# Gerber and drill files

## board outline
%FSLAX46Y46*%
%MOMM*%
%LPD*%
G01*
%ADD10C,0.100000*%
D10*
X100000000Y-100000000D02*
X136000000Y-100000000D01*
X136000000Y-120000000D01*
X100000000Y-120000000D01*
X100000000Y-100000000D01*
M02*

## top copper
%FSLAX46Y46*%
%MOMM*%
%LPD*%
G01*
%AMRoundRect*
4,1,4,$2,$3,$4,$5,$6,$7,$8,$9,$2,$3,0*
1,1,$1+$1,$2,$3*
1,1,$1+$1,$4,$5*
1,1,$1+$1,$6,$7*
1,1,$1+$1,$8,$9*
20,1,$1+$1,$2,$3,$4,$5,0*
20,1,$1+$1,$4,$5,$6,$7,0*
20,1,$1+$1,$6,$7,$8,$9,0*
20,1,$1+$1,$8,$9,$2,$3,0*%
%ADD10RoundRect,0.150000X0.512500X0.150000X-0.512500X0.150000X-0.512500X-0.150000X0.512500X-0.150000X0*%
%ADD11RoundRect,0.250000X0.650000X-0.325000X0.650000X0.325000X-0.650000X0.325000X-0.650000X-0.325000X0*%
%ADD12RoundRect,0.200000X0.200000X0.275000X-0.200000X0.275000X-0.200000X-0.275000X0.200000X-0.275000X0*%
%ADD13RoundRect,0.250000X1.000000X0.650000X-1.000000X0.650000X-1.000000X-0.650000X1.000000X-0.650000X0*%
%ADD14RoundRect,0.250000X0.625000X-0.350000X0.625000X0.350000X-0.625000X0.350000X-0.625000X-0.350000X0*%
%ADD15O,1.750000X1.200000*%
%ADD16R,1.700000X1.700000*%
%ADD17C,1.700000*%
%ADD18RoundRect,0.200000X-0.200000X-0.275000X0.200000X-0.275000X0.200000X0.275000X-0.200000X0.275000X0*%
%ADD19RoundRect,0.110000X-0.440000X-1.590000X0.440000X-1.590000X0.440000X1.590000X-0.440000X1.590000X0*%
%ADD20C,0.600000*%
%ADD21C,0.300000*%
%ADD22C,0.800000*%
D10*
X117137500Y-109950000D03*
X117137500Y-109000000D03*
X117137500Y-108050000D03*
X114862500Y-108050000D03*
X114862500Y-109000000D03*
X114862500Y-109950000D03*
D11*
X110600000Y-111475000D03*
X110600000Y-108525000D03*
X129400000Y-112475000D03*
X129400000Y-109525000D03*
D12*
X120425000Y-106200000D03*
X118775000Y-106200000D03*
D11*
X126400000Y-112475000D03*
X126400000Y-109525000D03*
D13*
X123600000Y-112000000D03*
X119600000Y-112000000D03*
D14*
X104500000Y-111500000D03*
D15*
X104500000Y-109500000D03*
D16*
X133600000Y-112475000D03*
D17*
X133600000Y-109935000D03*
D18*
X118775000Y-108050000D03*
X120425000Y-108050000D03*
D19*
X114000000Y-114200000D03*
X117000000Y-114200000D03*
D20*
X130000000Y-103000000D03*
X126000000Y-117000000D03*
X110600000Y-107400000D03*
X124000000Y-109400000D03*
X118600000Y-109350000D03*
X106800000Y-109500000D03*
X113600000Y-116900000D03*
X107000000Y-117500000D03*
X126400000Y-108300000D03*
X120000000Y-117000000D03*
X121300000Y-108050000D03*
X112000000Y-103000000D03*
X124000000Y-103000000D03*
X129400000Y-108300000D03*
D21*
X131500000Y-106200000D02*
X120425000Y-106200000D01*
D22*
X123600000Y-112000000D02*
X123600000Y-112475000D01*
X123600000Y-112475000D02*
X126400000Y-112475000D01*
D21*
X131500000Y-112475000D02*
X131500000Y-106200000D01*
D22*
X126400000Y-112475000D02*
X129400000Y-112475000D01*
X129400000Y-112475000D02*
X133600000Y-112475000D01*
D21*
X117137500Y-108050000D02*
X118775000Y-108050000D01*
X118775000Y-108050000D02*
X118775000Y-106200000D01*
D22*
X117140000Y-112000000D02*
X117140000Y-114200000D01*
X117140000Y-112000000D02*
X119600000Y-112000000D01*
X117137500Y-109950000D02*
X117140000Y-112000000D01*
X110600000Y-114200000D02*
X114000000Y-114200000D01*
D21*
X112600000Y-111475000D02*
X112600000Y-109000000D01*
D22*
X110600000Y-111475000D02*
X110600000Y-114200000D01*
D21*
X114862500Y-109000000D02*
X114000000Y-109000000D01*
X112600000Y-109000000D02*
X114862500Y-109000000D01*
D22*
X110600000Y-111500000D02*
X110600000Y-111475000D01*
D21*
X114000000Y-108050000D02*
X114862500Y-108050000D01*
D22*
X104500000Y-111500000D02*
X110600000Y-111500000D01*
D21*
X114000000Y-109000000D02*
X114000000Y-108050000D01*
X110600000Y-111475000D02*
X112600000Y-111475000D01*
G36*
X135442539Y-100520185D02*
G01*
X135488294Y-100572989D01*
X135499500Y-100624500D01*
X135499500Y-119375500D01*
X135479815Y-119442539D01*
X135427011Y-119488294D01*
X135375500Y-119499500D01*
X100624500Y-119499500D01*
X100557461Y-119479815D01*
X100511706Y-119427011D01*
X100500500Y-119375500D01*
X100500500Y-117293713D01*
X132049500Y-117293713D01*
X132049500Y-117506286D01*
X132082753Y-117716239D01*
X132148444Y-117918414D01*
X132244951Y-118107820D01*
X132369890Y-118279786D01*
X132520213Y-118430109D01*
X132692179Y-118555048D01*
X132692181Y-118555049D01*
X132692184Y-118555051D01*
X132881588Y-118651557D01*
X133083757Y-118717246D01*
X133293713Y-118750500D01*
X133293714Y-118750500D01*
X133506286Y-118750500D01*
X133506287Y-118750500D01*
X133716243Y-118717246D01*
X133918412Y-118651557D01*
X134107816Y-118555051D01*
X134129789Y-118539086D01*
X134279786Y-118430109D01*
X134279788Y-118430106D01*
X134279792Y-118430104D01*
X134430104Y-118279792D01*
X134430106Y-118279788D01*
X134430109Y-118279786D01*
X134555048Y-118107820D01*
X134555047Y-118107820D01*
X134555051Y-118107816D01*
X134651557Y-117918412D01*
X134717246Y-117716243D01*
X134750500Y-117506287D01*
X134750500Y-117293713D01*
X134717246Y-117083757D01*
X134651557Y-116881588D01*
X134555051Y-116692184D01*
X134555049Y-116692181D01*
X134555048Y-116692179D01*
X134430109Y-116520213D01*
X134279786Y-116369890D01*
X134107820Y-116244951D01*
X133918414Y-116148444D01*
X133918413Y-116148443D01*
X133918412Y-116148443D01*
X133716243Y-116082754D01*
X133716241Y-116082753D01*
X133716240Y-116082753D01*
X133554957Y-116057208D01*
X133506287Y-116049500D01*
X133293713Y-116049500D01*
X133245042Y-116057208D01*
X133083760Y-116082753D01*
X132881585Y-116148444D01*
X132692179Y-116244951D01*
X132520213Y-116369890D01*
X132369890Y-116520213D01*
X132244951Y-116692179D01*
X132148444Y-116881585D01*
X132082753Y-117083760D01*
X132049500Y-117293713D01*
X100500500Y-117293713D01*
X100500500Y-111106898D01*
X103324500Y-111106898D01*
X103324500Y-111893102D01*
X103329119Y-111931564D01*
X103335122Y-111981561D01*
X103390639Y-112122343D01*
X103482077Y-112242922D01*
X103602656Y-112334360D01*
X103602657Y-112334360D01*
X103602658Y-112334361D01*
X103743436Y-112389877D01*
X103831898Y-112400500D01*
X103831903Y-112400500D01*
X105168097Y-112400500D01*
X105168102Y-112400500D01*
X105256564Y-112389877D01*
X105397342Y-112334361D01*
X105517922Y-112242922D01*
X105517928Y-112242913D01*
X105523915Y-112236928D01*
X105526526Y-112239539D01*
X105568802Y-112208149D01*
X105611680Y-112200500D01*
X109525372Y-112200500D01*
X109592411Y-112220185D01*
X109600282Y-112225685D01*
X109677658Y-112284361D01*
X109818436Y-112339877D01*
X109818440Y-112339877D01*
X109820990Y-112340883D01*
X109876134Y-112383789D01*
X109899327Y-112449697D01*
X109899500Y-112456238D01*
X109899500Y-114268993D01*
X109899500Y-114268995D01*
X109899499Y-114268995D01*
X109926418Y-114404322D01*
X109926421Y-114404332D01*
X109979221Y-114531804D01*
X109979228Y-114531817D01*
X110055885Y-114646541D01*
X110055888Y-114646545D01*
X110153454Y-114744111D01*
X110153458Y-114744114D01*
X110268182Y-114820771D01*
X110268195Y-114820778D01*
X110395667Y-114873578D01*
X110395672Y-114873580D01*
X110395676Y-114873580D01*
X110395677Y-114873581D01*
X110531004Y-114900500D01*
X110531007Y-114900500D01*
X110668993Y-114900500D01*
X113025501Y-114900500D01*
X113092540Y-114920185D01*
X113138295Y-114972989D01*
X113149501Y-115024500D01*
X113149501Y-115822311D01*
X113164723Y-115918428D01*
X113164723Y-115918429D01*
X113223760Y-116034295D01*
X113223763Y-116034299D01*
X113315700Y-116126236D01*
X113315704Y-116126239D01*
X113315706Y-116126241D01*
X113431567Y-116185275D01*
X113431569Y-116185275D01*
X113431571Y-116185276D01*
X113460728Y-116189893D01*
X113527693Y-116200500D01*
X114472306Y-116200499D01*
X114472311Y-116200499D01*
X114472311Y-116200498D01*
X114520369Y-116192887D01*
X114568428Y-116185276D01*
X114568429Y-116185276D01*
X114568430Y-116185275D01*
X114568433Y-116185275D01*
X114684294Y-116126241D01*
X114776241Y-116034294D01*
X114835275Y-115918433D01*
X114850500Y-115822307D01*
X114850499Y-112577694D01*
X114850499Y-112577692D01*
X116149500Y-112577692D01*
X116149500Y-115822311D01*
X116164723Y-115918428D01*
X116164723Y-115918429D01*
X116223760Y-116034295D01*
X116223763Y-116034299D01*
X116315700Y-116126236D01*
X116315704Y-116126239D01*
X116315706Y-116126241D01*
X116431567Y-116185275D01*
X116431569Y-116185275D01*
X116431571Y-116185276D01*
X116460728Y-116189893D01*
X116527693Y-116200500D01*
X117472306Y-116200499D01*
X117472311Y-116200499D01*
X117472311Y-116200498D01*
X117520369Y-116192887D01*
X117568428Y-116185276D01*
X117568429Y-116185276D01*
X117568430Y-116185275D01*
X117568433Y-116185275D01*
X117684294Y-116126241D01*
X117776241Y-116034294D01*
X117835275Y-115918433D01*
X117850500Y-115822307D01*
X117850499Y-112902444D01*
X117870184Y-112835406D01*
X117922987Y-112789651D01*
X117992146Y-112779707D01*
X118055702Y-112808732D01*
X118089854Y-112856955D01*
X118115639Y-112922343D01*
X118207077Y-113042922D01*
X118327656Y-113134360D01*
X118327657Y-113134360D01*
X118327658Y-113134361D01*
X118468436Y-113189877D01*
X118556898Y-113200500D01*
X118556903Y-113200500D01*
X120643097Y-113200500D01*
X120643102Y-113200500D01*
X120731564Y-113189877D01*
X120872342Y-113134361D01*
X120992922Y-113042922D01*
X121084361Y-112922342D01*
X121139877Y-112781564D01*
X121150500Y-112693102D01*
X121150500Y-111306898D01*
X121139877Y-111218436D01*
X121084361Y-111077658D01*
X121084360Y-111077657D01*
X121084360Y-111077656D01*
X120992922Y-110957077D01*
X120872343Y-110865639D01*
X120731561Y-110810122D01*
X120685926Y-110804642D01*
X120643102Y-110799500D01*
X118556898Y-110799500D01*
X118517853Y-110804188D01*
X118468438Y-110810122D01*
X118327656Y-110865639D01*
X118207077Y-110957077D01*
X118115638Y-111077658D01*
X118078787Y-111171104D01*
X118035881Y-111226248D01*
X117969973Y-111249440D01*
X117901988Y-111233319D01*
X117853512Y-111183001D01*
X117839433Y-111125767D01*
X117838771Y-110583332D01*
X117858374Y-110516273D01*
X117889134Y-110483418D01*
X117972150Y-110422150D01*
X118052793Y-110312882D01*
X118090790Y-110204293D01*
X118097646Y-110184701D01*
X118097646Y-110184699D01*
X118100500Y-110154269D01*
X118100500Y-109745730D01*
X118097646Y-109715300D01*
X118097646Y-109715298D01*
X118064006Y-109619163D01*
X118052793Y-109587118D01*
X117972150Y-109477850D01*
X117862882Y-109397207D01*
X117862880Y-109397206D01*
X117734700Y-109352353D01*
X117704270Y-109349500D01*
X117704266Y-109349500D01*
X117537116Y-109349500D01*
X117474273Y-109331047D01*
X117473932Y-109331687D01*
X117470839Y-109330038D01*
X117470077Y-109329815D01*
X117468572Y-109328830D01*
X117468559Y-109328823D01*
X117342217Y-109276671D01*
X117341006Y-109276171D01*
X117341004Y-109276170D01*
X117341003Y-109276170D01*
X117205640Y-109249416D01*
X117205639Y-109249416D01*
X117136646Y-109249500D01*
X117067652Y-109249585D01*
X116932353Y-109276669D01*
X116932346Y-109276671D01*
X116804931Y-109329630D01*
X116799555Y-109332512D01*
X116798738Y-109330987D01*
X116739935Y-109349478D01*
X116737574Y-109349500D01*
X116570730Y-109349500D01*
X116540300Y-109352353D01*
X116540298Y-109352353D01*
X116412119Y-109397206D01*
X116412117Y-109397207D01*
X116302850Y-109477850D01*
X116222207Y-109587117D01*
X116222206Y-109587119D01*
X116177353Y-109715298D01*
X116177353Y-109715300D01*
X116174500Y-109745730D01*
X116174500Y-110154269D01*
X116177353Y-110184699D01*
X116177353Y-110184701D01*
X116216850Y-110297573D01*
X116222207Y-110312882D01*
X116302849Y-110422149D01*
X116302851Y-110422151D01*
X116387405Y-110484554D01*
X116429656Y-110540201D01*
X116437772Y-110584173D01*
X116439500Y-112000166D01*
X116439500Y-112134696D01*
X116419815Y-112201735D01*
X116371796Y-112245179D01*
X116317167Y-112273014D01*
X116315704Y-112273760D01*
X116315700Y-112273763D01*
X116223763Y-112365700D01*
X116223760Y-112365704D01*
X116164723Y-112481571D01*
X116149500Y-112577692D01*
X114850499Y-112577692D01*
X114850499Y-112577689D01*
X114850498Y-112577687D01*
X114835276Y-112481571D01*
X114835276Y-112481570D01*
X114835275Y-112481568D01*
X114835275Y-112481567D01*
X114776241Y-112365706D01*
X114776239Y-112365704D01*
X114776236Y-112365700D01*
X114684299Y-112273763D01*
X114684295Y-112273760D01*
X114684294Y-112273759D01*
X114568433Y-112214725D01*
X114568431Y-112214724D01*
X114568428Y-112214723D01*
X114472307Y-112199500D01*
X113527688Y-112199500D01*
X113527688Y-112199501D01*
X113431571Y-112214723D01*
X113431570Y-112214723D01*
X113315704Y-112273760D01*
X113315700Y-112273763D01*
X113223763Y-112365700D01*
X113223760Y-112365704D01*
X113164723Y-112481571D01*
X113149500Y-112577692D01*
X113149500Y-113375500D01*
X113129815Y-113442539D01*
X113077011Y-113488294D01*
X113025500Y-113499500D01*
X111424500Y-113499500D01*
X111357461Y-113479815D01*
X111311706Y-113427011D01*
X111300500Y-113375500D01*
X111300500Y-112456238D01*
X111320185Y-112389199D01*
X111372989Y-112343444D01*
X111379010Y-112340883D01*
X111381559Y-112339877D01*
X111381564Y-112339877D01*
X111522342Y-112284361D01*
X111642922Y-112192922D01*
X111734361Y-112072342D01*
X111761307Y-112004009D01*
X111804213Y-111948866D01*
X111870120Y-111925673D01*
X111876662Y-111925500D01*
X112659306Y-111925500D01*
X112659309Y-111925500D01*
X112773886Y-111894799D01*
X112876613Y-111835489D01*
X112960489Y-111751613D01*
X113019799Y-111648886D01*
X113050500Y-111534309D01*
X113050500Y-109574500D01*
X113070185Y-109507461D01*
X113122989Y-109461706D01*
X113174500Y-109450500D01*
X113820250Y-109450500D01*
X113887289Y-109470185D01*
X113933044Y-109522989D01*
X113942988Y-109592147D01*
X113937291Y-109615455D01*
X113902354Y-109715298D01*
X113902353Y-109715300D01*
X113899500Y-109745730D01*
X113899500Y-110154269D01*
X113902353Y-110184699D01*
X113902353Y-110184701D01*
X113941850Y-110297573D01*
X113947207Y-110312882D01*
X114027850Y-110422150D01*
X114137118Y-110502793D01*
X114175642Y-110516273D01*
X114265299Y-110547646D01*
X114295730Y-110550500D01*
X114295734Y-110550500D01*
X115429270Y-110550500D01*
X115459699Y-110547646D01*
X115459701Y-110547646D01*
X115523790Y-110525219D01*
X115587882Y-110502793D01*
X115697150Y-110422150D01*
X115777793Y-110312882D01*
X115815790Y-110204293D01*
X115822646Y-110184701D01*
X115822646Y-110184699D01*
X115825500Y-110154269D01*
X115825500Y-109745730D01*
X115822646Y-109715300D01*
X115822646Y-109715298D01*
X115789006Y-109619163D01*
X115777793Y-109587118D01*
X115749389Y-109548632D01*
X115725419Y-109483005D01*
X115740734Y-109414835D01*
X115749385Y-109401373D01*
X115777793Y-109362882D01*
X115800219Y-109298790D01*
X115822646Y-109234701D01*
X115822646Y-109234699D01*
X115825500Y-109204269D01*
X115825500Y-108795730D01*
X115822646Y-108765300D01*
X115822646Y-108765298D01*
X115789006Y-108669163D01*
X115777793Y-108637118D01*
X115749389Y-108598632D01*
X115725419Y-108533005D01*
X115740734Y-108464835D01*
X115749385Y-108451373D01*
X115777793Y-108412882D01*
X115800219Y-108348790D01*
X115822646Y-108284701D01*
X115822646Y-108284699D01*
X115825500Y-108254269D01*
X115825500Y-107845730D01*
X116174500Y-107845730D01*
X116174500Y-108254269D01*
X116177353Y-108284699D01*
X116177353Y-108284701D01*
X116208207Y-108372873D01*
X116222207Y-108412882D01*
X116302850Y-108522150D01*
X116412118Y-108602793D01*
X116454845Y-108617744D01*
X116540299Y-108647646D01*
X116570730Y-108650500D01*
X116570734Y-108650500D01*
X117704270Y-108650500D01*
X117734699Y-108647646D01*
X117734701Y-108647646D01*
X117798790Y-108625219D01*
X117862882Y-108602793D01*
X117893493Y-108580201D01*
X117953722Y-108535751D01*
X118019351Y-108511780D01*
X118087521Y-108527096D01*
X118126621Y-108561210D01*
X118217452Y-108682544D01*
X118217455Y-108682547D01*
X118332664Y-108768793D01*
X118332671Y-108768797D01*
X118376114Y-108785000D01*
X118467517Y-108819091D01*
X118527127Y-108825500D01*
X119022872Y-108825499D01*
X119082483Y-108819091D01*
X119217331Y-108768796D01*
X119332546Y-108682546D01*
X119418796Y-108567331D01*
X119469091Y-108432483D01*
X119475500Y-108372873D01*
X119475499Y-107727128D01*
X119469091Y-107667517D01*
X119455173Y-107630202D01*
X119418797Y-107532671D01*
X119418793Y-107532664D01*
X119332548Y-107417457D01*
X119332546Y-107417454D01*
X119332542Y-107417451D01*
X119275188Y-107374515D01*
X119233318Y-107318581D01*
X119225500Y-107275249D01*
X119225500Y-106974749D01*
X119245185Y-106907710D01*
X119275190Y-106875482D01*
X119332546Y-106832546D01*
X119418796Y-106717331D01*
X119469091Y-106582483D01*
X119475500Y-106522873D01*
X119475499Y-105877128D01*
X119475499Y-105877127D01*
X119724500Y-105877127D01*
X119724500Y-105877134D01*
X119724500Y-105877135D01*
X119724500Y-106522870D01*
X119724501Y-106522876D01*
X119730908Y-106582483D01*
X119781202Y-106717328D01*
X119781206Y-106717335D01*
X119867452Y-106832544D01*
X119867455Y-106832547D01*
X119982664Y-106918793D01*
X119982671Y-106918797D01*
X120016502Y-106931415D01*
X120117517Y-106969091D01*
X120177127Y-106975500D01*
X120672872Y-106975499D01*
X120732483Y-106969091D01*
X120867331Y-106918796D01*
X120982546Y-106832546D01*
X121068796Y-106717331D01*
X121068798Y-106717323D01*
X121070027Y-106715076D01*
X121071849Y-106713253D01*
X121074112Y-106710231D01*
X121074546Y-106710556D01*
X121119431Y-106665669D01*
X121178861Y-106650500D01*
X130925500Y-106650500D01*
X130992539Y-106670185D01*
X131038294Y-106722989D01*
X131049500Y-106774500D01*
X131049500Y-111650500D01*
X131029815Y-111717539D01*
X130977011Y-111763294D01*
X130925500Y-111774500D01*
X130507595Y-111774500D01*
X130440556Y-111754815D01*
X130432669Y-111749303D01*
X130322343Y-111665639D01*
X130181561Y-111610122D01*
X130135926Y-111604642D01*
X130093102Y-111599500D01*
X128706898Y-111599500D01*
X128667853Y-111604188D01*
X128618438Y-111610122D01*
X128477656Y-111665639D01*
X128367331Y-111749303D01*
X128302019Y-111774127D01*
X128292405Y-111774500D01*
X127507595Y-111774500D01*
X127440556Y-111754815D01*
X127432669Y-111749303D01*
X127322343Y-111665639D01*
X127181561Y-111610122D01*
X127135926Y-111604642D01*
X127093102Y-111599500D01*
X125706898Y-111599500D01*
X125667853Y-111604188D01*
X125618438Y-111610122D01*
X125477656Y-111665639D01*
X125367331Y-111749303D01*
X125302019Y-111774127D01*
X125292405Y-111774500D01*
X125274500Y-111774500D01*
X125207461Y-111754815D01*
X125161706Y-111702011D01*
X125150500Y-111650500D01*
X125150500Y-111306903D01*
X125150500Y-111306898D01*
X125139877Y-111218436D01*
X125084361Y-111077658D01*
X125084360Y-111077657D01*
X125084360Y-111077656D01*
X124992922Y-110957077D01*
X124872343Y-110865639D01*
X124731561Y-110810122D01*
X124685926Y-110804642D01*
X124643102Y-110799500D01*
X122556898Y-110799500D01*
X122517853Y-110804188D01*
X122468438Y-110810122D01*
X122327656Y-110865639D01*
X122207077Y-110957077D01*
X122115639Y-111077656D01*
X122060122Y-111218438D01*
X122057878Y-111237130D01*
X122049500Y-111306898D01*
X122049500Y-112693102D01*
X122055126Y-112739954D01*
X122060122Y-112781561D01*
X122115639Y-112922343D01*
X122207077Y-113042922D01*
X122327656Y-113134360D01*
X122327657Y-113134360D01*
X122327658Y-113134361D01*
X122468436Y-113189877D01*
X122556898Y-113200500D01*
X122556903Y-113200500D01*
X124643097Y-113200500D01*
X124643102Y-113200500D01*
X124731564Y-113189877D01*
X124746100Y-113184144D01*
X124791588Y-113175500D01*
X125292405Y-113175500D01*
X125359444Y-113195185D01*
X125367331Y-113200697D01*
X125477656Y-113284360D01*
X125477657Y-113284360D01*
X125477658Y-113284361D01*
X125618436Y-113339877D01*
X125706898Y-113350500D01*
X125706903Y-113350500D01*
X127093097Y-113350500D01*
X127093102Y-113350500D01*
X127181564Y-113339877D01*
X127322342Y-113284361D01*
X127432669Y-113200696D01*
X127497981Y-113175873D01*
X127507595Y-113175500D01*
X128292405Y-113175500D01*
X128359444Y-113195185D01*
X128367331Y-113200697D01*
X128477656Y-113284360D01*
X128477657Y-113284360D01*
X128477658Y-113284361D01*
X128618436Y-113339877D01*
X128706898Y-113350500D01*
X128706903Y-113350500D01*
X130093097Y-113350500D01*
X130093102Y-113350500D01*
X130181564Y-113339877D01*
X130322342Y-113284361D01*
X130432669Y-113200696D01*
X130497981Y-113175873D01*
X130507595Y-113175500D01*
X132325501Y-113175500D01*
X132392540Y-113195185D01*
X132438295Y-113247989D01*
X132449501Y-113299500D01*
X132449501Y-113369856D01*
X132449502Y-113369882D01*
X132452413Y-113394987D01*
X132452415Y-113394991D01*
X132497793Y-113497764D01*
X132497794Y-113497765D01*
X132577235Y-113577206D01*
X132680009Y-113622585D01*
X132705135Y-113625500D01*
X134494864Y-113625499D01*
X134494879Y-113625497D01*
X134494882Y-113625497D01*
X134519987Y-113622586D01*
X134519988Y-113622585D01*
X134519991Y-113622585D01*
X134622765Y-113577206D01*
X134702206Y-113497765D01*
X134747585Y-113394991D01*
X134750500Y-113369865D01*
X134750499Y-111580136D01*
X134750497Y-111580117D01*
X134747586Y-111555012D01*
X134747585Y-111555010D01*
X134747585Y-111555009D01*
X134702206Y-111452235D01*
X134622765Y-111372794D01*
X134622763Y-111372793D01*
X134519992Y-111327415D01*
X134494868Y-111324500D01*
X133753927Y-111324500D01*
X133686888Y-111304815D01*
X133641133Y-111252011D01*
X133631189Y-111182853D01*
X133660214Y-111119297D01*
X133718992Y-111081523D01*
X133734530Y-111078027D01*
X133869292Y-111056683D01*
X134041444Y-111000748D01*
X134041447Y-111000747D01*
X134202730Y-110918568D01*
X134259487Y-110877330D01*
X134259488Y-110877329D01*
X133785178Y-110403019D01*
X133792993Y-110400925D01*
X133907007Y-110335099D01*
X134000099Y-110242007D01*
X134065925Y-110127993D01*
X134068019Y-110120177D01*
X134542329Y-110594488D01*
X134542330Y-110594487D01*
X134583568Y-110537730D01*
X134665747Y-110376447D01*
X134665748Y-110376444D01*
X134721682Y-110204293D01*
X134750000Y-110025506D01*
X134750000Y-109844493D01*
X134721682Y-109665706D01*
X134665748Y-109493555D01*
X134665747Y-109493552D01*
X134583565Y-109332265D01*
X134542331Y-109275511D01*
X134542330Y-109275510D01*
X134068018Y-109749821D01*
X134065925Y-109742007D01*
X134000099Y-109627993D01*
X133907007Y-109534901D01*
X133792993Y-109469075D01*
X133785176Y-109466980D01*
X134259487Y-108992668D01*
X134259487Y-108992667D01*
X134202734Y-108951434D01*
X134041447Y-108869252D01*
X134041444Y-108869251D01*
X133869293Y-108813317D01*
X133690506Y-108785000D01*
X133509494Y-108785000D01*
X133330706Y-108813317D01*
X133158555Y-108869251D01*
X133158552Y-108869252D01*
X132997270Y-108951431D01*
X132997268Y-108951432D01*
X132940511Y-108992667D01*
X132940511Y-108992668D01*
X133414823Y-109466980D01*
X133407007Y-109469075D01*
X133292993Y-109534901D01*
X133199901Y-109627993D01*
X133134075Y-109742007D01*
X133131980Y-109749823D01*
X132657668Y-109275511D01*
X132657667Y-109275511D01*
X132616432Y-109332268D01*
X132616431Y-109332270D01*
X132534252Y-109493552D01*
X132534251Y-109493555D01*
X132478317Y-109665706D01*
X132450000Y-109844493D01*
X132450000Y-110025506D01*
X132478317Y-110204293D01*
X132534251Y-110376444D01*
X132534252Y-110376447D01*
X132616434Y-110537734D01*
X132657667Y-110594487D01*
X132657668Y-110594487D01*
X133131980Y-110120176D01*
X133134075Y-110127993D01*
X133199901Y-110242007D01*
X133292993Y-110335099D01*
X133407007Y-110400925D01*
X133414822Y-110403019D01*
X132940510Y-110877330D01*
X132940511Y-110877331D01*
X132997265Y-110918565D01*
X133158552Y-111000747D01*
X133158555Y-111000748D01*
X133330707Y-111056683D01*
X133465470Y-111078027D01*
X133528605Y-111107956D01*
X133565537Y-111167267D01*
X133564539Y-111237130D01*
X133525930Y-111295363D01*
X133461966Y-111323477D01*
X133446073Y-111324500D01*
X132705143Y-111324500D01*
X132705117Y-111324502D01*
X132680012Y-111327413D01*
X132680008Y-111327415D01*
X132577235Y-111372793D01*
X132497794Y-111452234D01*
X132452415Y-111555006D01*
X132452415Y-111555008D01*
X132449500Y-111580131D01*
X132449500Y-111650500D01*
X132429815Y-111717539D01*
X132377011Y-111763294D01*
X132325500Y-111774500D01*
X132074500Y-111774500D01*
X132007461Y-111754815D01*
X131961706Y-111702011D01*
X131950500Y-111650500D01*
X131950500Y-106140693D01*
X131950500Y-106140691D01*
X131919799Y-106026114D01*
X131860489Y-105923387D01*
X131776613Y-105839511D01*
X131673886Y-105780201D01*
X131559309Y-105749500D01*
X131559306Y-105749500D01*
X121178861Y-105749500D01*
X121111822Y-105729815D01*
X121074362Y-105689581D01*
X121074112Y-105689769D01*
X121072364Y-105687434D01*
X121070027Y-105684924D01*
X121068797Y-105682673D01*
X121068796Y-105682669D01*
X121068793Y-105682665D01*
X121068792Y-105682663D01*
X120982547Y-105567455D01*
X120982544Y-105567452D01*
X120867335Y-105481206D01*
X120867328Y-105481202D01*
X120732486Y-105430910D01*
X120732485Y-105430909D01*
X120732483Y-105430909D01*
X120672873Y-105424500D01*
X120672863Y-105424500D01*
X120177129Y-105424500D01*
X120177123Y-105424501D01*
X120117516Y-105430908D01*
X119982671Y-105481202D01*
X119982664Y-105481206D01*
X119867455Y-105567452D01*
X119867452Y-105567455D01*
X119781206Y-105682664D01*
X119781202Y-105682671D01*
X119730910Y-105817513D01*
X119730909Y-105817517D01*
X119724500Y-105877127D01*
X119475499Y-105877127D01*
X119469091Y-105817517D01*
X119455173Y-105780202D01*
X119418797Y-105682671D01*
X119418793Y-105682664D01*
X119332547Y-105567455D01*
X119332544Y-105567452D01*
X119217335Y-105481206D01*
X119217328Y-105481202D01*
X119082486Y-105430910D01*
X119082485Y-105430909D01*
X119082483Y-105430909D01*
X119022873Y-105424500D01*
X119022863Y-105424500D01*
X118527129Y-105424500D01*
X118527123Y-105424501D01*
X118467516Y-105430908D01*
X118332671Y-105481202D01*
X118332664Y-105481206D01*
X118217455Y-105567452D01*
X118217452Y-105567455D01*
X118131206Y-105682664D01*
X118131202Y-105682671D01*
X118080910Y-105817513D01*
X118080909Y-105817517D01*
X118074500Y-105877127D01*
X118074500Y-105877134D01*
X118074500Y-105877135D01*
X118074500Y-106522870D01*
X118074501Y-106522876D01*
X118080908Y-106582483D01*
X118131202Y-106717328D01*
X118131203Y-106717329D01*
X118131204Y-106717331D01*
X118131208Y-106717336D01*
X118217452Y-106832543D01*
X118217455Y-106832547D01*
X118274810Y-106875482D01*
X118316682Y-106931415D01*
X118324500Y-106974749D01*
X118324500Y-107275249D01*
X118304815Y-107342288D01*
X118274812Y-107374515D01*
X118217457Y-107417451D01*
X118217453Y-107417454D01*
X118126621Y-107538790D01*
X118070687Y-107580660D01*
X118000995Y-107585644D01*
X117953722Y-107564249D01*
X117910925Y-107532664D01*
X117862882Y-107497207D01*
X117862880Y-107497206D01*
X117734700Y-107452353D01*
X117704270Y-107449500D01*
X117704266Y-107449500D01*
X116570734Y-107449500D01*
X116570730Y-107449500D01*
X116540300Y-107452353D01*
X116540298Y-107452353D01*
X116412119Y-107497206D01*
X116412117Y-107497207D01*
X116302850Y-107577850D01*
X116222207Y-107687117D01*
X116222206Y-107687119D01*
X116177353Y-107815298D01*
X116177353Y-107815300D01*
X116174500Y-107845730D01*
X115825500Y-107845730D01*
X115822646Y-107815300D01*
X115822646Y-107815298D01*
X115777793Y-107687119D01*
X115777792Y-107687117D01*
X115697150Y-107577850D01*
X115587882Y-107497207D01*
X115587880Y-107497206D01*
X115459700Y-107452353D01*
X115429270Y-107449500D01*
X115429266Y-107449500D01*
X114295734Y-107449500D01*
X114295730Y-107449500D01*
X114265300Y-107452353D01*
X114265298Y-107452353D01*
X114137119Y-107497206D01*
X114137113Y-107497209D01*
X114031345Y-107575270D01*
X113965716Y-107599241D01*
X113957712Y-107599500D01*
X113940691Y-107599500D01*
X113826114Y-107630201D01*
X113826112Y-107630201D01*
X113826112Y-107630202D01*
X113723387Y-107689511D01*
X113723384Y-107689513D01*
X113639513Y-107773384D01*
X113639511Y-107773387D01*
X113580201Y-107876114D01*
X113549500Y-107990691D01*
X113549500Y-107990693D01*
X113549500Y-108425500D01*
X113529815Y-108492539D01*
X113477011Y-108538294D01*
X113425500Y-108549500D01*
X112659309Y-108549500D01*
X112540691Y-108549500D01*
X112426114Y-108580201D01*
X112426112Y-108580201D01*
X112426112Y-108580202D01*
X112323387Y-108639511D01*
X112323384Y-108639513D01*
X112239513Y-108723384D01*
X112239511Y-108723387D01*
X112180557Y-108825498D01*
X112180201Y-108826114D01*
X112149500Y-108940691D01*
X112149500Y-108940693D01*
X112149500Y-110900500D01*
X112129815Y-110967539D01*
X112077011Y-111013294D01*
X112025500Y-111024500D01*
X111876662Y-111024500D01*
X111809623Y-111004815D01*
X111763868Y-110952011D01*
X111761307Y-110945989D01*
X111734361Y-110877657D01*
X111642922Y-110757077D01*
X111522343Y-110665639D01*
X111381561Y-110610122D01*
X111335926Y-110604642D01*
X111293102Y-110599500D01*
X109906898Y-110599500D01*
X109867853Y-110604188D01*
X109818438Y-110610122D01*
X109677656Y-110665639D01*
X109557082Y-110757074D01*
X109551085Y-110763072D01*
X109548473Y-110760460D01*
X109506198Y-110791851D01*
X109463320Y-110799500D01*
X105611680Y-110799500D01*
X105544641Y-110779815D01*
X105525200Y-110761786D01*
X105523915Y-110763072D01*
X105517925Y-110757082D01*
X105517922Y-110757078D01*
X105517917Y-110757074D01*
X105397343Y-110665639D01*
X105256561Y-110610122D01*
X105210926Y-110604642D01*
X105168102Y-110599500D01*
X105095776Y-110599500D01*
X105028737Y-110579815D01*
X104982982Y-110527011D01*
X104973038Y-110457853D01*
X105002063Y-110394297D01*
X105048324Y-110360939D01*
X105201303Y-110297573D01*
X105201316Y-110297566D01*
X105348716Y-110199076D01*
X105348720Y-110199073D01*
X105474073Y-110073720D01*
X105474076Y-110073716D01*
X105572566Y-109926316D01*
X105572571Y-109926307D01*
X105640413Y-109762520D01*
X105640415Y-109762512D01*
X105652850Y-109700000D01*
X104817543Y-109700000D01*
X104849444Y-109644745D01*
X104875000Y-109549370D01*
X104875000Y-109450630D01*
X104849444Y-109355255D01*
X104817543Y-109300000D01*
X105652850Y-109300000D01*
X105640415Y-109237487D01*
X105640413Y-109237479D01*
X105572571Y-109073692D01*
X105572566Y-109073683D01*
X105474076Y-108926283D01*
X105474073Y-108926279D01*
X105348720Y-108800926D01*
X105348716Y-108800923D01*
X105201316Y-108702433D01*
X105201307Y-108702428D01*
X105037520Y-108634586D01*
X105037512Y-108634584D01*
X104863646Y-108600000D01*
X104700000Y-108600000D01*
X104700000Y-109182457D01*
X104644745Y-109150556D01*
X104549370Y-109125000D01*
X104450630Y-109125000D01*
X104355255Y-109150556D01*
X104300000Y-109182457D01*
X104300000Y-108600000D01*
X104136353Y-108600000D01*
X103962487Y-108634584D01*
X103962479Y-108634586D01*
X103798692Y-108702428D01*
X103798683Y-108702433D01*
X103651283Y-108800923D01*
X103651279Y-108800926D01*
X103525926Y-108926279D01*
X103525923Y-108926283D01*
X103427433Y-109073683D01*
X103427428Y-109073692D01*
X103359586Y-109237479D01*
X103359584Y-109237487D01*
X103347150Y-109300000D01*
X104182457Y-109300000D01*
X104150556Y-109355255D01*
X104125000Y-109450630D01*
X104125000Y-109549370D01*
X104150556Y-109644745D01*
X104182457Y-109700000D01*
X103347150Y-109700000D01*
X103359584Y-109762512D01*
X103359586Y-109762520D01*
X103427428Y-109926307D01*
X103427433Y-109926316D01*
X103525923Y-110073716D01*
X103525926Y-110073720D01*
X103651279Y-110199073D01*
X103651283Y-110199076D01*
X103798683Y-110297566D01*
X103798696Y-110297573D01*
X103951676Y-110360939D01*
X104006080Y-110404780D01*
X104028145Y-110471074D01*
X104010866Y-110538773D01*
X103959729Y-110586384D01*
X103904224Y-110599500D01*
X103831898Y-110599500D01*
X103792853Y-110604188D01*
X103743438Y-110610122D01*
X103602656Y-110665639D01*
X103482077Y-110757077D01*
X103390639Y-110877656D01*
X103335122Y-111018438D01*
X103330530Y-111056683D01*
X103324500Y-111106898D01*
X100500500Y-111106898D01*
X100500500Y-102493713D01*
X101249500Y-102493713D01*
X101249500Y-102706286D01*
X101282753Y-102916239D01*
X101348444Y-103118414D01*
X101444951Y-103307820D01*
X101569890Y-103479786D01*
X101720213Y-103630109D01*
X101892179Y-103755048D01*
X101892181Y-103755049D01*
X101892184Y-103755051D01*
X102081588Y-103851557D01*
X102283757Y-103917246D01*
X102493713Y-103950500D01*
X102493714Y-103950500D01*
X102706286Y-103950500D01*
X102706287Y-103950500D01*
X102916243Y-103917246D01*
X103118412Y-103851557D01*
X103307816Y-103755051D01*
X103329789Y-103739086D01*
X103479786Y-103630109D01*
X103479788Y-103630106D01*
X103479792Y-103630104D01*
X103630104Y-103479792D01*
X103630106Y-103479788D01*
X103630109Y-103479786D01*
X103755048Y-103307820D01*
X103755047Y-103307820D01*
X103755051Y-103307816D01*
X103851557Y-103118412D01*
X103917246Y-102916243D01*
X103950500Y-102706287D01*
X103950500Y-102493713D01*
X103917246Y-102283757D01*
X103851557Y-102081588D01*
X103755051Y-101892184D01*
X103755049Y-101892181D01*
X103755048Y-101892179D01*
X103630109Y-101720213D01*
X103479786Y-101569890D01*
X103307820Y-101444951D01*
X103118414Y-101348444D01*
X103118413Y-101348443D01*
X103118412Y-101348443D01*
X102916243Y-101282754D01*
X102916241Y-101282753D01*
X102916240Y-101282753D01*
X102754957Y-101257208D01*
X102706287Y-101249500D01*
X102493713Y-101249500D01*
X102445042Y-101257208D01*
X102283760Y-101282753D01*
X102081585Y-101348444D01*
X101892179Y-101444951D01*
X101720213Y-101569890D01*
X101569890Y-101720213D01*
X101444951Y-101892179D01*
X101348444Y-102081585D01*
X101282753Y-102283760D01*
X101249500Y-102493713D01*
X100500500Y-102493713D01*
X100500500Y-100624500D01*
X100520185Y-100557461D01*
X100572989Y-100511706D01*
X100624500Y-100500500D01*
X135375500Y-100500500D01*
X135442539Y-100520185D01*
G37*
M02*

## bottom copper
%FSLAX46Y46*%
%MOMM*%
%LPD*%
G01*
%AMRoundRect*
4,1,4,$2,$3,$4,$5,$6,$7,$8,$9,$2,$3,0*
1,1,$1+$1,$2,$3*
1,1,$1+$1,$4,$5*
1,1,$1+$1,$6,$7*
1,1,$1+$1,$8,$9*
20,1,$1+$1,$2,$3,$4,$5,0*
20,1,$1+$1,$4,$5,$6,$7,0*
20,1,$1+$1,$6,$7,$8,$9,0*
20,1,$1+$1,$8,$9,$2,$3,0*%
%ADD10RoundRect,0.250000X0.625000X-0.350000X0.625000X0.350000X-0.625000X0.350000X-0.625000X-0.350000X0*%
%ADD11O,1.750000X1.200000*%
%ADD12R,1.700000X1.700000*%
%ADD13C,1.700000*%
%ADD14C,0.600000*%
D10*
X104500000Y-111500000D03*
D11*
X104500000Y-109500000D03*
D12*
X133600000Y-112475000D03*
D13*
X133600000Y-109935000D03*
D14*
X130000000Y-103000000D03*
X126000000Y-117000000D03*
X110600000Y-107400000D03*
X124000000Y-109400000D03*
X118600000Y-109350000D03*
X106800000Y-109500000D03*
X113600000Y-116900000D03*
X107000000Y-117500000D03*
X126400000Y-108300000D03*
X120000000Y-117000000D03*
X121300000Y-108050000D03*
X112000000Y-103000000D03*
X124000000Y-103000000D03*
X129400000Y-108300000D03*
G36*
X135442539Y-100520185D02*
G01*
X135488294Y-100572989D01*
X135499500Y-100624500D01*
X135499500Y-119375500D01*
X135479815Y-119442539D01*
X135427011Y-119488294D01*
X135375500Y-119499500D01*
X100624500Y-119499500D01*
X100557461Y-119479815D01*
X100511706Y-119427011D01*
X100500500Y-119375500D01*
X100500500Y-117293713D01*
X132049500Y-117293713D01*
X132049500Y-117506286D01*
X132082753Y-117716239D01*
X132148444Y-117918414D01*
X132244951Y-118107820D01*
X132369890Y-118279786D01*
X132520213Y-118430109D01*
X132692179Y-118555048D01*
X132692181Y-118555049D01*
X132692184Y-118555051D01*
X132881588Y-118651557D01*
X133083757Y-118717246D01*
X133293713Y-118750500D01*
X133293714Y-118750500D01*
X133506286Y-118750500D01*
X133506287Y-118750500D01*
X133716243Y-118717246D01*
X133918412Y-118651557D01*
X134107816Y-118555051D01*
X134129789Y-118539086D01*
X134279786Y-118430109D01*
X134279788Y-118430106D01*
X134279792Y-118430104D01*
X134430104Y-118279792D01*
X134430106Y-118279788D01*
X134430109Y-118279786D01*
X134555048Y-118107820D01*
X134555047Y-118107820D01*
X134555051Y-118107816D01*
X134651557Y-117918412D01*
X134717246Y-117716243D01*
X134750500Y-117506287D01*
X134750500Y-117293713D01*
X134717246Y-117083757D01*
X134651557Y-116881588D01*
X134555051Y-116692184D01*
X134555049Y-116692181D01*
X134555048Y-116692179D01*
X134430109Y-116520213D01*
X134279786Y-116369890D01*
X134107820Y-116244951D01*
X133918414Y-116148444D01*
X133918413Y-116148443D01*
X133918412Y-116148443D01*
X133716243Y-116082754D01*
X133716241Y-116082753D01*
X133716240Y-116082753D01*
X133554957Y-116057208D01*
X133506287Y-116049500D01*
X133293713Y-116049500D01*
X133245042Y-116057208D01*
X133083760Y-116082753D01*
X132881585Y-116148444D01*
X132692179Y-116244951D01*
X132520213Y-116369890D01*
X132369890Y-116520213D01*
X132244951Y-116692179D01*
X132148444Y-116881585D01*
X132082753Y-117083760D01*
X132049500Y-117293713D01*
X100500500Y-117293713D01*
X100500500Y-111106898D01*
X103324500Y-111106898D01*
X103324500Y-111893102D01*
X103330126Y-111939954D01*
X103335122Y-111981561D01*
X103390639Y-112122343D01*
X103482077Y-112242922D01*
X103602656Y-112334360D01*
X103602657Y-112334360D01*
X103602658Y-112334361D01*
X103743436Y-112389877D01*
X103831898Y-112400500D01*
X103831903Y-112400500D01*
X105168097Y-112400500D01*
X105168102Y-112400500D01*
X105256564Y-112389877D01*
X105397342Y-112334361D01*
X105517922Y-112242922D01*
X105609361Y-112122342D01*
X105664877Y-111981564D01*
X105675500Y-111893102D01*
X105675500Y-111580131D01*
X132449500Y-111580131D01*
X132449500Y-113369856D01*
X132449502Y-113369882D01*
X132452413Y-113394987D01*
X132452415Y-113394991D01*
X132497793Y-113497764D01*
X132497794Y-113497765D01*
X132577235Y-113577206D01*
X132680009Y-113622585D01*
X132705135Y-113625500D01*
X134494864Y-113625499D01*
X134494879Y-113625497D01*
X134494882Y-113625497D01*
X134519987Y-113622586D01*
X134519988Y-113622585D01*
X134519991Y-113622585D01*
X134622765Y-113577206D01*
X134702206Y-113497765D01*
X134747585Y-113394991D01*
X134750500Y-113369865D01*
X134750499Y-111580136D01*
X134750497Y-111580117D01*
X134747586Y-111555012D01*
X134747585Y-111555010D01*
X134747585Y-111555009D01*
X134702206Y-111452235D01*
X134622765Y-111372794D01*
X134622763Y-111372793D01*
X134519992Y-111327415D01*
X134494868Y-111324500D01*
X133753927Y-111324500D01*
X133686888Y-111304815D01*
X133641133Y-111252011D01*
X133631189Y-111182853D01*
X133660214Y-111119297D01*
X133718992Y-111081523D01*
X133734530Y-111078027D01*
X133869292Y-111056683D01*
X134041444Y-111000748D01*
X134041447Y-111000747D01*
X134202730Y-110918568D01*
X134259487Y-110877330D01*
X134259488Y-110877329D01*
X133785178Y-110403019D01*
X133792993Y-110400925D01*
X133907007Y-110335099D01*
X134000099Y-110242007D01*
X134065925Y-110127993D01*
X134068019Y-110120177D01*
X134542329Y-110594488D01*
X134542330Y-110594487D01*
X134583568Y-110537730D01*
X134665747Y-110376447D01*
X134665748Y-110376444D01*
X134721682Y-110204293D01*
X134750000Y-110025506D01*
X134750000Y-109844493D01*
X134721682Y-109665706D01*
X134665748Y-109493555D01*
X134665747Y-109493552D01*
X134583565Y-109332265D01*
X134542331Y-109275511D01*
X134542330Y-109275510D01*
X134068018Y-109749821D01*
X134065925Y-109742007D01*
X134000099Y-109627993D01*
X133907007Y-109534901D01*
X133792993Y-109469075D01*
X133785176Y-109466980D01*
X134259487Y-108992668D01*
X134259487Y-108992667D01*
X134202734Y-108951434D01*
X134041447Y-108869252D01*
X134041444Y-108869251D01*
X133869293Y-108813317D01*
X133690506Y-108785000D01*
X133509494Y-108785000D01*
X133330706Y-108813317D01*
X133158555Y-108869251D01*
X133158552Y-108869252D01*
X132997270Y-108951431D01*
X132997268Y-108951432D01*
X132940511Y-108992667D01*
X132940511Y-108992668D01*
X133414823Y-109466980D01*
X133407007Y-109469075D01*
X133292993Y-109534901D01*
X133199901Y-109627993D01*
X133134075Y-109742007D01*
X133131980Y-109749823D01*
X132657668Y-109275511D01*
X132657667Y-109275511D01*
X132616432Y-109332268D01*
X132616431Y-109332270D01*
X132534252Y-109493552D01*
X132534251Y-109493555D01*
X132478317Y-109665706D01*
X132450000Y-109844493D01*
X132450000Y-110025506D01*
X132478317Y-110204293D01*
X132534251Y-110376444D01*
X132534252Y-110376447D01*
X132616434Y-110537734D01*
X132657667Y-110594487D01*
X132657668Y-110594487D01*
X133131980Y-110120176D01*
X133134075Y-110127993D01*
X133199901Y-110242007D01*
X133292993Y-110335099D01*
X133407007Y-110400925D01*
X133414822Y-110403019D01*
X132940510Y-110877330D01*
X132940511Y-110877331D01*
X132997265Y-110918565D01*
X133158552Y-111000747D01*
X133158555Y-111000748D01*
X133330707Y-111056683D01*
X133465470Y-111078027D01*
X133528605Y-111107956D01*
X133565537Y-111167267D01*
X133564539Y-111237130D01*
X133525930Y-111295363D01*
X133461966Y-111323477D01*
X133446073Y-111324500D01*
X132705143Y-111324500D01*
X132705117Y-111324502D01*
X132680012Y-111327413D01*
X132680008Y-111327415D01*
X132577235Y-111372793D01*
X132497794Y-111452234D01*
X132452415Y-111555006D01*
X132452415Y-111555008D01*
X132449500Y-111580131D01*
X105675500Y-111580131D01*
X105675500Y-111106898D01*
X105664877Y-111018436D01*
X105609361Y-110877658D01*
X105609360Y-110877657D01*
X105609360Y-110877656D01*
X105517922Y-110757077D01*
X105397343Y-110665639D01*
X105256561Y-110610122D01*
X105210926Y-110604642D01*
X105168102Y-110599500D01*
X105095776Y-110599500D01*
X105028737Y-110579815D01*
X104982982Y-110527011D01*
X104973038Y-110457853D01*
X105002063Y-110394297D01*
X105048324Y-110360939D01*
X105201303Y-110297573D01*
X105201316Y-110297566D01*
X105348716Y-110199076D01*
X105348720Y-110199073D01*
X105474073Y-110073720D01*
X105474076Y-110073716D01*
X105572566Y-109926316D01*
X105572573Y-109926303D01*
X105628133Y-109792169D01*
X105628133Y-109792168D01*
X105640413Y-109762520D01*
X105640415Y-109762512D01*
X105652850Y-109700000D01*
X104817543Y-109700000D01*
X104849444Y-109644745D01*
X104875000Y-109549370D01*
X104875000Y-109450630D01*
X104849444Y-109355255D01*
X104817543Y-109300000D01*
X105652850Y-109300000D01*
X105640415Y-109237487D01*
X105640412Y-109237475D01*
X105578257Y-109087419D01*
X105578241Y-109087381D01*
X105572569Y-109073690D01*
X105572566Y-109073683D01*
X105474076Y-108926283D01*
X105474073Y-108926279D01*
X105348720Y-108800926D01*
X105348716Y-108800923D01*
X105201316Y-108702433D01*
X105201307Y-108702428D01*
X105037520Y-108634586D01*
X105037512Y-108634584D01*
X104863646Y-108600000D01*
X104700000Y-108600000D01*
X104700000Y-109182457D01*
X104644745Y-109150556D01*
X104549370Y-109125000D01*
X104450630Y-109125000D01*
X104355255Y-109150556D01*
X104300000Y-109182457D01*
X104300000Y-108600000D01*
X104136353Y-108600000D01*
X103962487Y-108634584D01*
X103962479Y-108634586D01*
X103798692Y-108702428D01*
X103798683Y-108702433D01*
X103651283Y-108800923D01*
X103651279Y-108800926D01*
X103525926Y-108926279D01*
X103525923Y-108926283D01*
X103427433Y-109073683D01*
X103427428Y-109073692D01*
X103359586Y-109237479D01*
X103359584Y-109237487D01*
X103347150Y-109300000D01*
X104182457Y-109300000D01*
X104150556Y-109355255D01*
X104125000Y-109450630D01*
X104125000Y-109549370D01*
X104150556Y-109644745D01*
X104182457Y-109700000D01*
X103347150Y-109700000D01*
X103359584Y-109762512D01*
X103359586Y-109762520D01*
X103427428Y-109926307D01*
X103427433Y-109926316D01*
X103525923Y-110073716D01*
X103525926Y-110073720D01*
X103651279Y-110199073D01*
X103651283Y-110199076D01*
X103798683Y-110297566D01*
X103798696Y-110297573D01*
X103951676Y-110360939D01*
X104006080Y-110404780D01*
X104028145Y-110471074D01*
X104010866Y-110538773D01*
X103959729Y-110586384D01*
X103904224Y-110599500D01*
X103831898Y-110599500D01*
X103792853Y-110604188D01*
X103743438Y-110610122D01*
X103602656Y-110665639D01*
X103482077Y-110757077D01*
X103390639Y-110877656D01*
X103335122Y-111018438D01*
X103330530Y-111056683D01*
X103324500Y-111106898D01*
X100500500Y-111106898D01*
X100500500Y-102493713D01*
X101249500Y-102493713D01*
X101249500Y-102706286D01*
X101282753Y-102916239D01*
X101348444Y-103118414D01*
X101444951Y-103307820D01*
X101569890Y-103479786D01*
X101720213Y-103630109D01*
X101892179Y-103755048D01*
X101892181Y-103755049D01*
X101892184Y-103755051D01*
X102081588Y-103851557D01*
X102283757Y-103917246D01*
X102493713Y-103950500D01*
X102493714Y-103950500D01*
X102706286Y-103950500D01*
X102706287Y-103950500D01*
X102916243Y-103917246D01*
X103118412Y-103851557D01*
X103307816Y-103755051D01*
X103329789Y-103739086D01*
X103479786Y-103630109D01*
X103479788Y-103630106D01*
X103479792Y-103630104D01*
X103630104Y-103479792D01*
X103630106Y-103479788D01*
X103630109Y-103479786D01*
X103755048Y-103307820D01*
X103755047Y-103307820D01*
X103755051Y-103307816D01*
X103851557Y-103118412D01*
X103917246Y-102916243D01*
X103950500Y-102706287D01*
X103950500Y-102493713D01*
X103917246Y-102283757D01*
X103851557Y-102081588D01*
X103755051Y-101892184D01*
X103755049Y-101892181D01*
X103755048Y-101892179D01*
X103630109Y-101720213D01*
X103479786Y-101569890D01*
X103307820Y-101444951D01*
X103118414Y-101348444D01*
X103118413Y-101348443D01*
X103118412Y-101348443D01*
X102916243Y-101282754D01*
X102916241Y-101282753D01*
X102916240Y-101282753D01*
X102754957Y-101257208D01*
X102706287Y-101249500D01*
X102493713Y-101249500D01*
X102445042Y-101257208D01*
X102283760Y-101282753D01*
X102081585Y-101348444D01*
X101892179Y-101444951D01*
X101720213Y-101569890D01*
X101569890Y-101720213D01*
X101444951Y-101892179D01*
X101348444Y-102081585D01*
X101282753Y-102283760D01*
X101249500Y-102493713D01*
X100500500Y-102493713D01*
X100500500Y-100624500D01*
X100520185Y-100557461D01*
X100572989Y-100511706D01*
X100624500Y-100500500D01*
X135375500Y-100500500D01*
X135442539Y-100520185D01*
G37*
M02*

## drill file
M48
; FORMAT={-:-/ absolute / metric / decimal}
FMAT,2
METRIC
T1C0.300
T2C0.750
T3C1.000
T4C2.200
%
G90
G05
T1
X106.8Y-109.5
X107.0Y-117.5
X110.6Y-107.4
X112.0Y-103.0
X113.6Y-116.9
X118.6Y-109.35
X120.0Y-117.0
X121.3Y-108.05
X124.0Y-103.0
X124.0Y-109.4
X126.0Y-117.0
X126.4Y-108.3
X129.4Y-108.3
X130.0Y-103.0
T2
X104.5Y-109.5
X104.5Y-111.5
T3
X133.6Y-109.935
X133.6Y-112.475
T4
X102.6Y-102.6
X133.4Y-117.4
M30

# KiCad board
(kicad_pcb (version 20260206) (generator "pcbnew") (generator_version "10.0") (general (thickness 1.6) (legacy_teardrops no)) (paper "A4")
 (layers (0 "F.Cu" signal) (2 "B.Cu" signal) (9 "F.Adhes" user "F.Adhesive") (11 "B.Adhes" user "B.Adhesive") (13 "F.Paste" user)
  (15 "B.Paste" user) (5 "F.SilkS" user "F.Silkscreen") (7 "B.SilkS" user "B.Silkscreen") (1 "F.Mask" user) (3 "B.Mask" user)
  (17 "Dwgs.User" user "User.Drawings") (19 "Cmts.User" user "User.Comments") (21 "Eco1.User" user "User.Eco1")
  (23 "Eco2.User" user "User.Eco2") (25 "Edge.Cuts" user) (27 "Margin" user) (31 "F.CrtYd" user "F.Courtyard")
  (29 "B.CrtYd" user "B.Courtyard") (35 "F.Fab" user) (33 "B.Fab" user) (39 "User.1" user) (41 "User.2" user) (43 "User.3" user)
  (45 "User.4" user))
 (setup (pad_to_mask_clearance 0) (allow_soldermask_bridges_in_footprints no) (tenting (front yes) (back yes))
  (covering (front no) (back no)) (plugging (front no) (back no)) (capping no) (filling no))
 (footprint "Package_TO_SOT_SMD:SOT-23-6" (layer "F.Cu") (at 116 109 180)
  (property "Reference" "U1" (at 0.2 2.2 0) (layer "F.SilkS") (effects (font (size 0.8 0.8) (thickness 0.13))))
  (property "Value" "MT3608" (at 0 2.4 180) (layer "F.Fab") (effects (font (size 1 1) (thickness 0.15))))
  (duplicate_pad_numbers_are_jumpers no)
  (pad "1" smd roundrect (at -1.1375 -0.95 180) (size 1.325 0.6) (layers "F.Cu" "F.Mask" "F.Paste") (roundrect_rratio 0.25) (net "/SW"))
  (pad "2" smd roundrect (at -1.1375 0 180) (size 1.325 0.6) (layers "F.Cu" "F.Mask" "F.Paste") (roundrect_rratio 0.25) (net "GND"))
  (pad "3" smd roundrect (at -1.1375 0.95 180) (size 1.325 0.6) (layers "F.Cu" "F.Mask" "F.Paste") (roundrect_rratio 0.25) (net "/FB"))
  (pad "4" smd roundrect (at 1.1375 0.95 180) (size 1.325 0.6) (layers "F.Cu" "F.Mask" "F.Paste") (roundrect_rratio 0.25) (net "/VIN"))
  (pad "5" smd roundrect (at 1.1375 0 180) (size 1.325 0.6) (layers "F.Cu" "F.Mask" "F.Paste") (roundrect_rratio 0.25) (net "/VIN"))
  (pad "6" smd roundrect (at 1.1375 -0.95 180) (size 1.325 0.6) (layers "F.Cu" "F.Mask" "F.Paste") (roundrect_rratio 0.25)
   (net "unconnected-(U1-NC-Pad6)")))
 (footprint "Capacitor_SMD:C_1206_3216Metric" (layer "F.Cu") (at 110.6 110 90)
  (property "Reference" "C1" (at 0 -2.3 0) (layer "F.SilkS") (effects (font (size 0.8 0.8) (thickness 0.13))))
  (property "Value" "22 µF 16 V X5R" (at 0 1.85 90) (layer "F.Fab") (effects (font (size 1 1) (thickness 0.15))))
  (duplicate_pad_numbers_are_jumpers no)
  (pad "1" smd roundrect (at -1.475 0 90) (size 1.15 1.8) (layers "F.Cu" "F.Mask" "F.Paste") (roundrect_rratio 0.217391) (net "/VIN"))
  (pad "2" smd roundrect (at 1.475 0 90) (size 1.15 1.8) (layers "F.Cu" "F.Mask" "F.Paste") (roundrect_rratio 0.217391) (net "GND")))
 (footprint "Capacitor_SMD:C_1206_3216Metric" (layer "F.Cu") (at 129.4 111 90)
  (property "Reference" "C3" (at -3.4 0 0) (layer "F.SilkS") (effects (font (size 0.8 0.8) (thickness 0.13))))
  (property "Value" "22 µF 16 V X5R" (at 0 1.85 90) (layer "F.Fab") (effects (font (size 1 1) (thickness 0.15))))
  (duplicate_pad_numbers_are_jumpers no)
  (pad "1" smd roundrect (at -1.475 0 90) (size 1.15 1.8) (layers "F.Cu" "F.Mask" "F.Paste") (roundrect_rratio 0.217391) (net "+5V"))
  (pad "2" smd roundrect (at 1.475 0 90) (size 1.15 1.8) (layers "F.Cu" "F.Mask" "F.Paste") (roundrect_rratio 0.217391) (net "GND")))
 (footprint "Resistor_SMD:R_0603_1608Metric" (layer "F.Cu") (at 119.6 106.2 180)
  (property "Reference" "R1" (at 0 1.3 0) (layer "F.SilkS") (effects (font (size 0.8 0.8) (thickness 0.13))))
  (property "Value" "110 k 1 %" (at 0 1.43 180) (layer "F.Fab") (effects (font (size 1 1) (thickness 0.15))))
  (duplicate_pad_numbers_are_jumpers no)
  (pad "1" smd roundrect (at -0.825 0 180) (size 0.8 0.95) (layers "F.Cu" "F.Mask" "F.Paste") (roundrect_rratio 0.25) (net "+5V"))
  (pad "2" smd roundrect (at 0.825 0 180) (size 0.8 0.95) (layers "F.Cu" "F.Mask" "F.Paste") (roundrect_rratio 0.25) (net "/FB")))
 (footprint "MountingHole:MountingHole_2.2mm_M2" (layer "F.Cu") (at 133.4 117.4)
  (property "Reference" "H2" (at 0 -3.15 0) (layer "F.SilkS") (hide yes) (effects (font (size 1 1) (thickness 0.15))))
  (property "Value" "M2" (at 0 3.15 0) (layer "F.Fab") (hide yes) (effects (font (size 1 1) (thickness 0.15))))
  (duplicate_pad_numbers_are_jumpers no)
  (pad "" np_thru_hole circle (at 0 0) (size 2.2 2.2) (drill 2.2) (layers "*.Cu" "*.Mask")))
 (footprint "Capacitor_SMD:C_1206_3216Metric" (layer "F.Cu") (at 126.4 111 90)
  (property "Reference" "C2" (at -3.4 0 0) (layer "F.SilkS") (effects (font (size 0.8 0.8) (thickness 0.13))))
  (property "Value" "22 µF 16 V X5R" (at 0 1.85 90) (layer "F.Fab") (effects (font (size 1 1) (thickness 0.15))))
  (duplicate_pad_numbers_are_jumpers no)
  (pad "1" smd roundrect (at -1.475 0 90) (size 1.15 1.8) (layers "F.Cu" "F.Mask" "F.Paste") (roundrect_rratio 0.217391) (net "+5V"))
  (pad "2" smd roundrect (at 1.475 0 90) (size 1.15 1.8) (layers "F.Cu" "F.Mask" "F.Paste") (roundrect_rratio 0.217391) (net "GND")))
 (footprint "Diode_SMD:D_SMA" (layer "F.Cu") (at 121.6 112 180)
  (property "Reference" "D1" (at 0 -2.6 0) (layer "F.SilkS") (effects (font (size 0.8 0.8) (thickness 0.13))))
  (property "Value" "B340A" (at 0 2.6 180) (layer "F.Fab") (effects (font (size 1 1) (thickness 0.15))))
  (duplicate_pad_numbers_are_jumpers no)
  (pad "1" smd roundrect (at -2 0 180) (size 2.5 1.8) (layers "F.Cu" "F.Mask" "F.Paste") (roundrect_rratio 0.1388888889) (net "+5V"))
  (pad "2" smd roundrect (at 2 0 180) (size 2.5 1.8) (layers "F.Cu" "F.Mask" "F.Paste") (roundrect_rratio 0.1388888889) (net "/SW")))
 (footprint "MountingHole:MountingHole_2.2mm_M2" (layer "F.Cu") (at 102.6 102.6)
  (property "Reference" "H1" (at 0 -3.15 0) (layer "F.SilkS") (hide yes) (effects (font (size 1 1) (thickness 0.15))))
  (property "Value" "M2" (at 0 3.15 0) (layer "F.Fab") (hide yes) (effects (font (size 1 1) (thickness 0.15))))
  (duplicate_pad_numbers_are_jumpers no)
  (pad "" np_thru_hole circle (at 0 0) (size 2.2 2.2) (drill 2.2) (layers "*.Cu" "*.Mask")))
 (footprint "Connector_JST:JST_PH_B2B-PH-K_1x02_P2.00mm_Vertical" (layer "F.Cu") (at 104.5 111.5 90)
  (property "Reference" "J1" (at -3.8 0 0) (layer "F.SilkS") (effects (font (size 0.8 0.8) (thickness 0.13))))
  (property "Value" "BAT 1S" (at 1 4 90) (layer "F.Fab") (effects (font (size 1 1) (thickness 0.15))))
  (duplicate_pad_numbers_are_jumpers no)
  (pad "1" thru_hole roundrect (at 0 0 90) (size 1.2 1.75) (drill 0.75) (layers "*.Cu" "*.Mask") (remove_unused_layers no)
   (roundrect_rratio 0.208333) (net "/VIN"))
  (pad "2" thru_hole oval (at 2 0 90) (size 1.2 1.75) (drill 0.75) (layers "*.Cu" "*.Mask") (remove_unused_layers no) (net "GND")))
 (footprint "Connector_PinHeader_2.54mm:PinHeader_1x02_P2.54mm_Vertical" (layer "F.Cu") (at 133.6 112.475 180)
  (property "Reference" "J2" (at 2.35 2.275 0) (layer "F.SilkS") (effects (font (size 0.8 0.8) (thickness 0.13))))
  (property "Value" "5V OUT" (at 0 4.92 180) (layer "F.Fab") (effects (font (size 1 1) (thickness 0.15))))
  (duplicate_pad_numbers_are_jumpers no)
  (pad "1" thru_hole rect (at 0 0 180) (size 1.7 1.7) (drill 1) (layers "*.Cu" "*.Mask") (remove_unused_layers no) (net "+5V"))
  (pad "2" thru_hole circle (at 0 2.54 180) (size 1.7 1.7) (drill 1) (layers "*.Cu" "*.Mask") (remove_unused_layers no) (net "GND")))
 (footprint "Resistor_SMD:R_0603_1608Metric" (layer "F.Cu") (at 119.6 108.05)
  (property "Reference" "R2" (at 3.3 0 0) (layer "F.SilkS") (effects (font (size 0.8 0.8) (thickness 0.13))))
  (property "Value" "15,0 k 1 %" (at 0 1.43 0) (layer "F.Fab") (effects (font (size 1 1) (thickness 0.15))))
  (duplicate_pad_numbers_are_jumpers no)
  (pad "1" smd roundrect (at -0.825 0) (size 0.8 0.95) (layers "F.Cu" "F.Mask" "F.Paste") (roundrect_rratio 0.25) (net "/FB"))
  (pad "2" smd roundrect (at 0.825 0) (size 0.8 0.95) (layers "F.Cu" "F.Mask" "F.Paste") (roundrect_rratio 0.25) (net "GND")))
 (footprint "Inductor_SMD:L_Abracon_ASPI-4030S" (layer "F.Cu") (at 115.5 114.2)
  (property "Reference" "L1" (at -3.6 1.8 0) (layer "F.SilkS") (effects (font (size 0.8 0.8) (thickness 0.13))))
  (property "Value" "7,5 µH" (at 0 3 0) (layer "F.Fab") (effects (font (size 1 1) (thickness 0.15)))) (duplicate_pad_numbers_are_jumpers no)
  (pad "1" smd roundrect (at -1.5 0) (size 1.1 3.4) (layers "F.Cu" "F.Mask" "F.Paste") (roundrect_rratio 0.1) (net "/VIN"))
  (pad "2" smd roundrect (at 1.5 0) (size 1.1 3.4) (layers "F.Cu" "F.Mask" "F.Paste") (roundrect_rratio 0.1) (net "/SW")))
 (gr_rect (start 100 100) (end 136 120) (stroke (width 0.1) (type default)) (fill no) (layer "Edge.Cuts"))
 (segment (start 131.5 106.2) (end 120.425 106.2) (width 0.3) (layer "F.Cu") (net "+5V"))
 (segment (start 123.6 112) (end 123.6 112.475) (width 0.8) (layer "F.Cu") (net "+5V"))
 (segment (start 123.6 112.475) (end 126.4 112.475) (width 0.8) (layer "F.Cu") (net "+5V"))
 (segment (start 131.5 112.475) (end 131.5 106.2) (width 0.3) (layer "F.Cu") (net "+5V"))
 (segment (start 126.4 112.475) (end 129.4 112.475) (width 0.8) (layer "F.Cu") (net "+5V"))
 (segment (start 129.4 112.475) (end 133.6 112.475) (width 0.8) (layer "F.Cu") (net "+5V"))
 (segment (start 117.1375 108.05) (end 118.775 108.05) (width 0.3) (layer "F.Cu") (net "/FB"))
 (segment (start 118.775 108.05) (end 118.775 106.2) (width 0.3) (layer "F.Cu") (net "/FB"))
 (segment (start 117.14 112) (end 117.14 114.2) (width 0.8) (layer "F.Cu") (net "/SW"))
 (segment (start 117.14 112) (end 119.6 112) (width 0.8) (layer "F.Cu") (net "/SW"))
 (segment (start 117.1375 109.95) (end 117.14 112) (width 0.8) (layer "F.Cu") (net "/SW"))
 (segment (start 110.6 114.2) (end 114 114.2) (width 0.8) (layer "F.Cu") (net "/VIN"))
 (segment (start 112.6 111.475) (end 112.6 109) (width 0.3) (layer "F.Cu") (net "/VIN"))
 (segment (start 110.6 111.475) (end 110.6 114.2) (width 0.8) (layer "F.Cu") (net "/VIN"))
 (segment (start 114.8625 109) (end 114 109) (width 0.3) (layer "F.Cu") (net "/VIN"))
 (segment (start 112.6 109) (end 114.8625 109) (width 0.3) (layer "F.Cu") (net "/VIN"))
 (segment (start 110.6 111.5) (end 110.6 111.475) (width 0.8) (layer "F.Cu") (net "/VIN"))
 (segment (start 114 108.05) (end 114.8625 108.05) (width 0.3) (layer "F.Cu") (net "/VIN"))
 (segment (start 104.5 111.5) (end 110.6 111.5) (width 0.8) (layer "F.Cu") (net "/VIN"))
 (segment (start 114 109) (end 114 108.05) (width 0.3) (layer "F.Cu") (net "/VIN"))
 (segment (start 110.6 111.475) (end 112.6 111.475) (width 0.3) (layer "F.Cu") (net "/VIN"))
 (via (at 130 103) (size 0.6) (drill 0.3) (layers "F.Cu" "B.Cu") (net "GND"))
 (via (at 126 117) (size 0.6) (drill 0.3) (layers "F.Cu" "B.Cu") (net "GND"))
 (via (at 110.6 107.4) (size 0.6) (drill 0.3) (layers "F.Cu" "B.Cu") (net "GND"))
 (via (at 124 109.4) (size 0.6) (drill 0.3) (layers "F.Cu" "B.Cu") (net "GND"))
 (via (at 118.6 109.35) (size 0.6) (drill 0.3) (layers "F.Cu" "B.Cu") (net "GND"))
 (via (at 106.8 109.5) (size 0.6) (drill 0.3) (layers "F.Cu" "B.Cu") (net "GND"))
 (via (at 113.6 116.9) (size 0.6) (drill 0.3) (layers "F.Cu" "B.Cu") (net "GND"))
 (via (at 107 117.5) (size 0.6) (drill 0.3) (layers "F.Cu" "B.Cu") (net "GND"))
 (via (at 126.4 108.3) (size 0.6) (drill 0.3) (layers "F.Cu" "B.Cu") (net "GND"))
 (via (at 120 117) (size 0.6) (drill 0.3) (layers "F.Cu" "B.Cu") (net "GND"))
 (via (at 121.3 108.05) (size 0.6) (drill 0.3) (layers "F.Cu" "B.Cu") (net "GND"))
 (via (at 112 103) (size 0.6) (drill 0.3) (layers "F.Cu" "B.Cu") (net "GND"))
 (via (at 124 103) (size 0.6) (drill 0.3) (layers "F.Cu" "B.Cu") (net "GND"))
 (via (at 129.4 108.3) (size 0.6) (drill 0.3) (layers "F.Cu" "B.Cu") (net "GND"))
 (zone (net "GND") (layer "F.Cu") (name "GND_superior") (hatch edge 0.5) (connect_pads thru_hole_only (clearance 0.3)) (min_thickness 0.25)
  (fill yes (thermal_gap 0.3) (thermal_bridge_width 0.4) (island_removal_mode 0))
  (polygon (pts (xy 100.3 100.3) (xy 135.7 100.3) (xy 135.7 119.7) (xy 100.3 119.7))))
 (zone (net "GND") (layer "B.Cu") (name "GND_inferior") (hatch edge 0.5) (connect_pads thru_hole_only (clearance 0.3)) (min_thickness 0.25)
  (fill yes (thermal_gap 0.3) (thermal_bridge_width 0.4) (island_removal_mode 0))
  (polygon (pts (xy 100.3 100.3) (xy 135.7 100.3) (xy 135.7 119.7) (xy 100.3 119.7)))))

